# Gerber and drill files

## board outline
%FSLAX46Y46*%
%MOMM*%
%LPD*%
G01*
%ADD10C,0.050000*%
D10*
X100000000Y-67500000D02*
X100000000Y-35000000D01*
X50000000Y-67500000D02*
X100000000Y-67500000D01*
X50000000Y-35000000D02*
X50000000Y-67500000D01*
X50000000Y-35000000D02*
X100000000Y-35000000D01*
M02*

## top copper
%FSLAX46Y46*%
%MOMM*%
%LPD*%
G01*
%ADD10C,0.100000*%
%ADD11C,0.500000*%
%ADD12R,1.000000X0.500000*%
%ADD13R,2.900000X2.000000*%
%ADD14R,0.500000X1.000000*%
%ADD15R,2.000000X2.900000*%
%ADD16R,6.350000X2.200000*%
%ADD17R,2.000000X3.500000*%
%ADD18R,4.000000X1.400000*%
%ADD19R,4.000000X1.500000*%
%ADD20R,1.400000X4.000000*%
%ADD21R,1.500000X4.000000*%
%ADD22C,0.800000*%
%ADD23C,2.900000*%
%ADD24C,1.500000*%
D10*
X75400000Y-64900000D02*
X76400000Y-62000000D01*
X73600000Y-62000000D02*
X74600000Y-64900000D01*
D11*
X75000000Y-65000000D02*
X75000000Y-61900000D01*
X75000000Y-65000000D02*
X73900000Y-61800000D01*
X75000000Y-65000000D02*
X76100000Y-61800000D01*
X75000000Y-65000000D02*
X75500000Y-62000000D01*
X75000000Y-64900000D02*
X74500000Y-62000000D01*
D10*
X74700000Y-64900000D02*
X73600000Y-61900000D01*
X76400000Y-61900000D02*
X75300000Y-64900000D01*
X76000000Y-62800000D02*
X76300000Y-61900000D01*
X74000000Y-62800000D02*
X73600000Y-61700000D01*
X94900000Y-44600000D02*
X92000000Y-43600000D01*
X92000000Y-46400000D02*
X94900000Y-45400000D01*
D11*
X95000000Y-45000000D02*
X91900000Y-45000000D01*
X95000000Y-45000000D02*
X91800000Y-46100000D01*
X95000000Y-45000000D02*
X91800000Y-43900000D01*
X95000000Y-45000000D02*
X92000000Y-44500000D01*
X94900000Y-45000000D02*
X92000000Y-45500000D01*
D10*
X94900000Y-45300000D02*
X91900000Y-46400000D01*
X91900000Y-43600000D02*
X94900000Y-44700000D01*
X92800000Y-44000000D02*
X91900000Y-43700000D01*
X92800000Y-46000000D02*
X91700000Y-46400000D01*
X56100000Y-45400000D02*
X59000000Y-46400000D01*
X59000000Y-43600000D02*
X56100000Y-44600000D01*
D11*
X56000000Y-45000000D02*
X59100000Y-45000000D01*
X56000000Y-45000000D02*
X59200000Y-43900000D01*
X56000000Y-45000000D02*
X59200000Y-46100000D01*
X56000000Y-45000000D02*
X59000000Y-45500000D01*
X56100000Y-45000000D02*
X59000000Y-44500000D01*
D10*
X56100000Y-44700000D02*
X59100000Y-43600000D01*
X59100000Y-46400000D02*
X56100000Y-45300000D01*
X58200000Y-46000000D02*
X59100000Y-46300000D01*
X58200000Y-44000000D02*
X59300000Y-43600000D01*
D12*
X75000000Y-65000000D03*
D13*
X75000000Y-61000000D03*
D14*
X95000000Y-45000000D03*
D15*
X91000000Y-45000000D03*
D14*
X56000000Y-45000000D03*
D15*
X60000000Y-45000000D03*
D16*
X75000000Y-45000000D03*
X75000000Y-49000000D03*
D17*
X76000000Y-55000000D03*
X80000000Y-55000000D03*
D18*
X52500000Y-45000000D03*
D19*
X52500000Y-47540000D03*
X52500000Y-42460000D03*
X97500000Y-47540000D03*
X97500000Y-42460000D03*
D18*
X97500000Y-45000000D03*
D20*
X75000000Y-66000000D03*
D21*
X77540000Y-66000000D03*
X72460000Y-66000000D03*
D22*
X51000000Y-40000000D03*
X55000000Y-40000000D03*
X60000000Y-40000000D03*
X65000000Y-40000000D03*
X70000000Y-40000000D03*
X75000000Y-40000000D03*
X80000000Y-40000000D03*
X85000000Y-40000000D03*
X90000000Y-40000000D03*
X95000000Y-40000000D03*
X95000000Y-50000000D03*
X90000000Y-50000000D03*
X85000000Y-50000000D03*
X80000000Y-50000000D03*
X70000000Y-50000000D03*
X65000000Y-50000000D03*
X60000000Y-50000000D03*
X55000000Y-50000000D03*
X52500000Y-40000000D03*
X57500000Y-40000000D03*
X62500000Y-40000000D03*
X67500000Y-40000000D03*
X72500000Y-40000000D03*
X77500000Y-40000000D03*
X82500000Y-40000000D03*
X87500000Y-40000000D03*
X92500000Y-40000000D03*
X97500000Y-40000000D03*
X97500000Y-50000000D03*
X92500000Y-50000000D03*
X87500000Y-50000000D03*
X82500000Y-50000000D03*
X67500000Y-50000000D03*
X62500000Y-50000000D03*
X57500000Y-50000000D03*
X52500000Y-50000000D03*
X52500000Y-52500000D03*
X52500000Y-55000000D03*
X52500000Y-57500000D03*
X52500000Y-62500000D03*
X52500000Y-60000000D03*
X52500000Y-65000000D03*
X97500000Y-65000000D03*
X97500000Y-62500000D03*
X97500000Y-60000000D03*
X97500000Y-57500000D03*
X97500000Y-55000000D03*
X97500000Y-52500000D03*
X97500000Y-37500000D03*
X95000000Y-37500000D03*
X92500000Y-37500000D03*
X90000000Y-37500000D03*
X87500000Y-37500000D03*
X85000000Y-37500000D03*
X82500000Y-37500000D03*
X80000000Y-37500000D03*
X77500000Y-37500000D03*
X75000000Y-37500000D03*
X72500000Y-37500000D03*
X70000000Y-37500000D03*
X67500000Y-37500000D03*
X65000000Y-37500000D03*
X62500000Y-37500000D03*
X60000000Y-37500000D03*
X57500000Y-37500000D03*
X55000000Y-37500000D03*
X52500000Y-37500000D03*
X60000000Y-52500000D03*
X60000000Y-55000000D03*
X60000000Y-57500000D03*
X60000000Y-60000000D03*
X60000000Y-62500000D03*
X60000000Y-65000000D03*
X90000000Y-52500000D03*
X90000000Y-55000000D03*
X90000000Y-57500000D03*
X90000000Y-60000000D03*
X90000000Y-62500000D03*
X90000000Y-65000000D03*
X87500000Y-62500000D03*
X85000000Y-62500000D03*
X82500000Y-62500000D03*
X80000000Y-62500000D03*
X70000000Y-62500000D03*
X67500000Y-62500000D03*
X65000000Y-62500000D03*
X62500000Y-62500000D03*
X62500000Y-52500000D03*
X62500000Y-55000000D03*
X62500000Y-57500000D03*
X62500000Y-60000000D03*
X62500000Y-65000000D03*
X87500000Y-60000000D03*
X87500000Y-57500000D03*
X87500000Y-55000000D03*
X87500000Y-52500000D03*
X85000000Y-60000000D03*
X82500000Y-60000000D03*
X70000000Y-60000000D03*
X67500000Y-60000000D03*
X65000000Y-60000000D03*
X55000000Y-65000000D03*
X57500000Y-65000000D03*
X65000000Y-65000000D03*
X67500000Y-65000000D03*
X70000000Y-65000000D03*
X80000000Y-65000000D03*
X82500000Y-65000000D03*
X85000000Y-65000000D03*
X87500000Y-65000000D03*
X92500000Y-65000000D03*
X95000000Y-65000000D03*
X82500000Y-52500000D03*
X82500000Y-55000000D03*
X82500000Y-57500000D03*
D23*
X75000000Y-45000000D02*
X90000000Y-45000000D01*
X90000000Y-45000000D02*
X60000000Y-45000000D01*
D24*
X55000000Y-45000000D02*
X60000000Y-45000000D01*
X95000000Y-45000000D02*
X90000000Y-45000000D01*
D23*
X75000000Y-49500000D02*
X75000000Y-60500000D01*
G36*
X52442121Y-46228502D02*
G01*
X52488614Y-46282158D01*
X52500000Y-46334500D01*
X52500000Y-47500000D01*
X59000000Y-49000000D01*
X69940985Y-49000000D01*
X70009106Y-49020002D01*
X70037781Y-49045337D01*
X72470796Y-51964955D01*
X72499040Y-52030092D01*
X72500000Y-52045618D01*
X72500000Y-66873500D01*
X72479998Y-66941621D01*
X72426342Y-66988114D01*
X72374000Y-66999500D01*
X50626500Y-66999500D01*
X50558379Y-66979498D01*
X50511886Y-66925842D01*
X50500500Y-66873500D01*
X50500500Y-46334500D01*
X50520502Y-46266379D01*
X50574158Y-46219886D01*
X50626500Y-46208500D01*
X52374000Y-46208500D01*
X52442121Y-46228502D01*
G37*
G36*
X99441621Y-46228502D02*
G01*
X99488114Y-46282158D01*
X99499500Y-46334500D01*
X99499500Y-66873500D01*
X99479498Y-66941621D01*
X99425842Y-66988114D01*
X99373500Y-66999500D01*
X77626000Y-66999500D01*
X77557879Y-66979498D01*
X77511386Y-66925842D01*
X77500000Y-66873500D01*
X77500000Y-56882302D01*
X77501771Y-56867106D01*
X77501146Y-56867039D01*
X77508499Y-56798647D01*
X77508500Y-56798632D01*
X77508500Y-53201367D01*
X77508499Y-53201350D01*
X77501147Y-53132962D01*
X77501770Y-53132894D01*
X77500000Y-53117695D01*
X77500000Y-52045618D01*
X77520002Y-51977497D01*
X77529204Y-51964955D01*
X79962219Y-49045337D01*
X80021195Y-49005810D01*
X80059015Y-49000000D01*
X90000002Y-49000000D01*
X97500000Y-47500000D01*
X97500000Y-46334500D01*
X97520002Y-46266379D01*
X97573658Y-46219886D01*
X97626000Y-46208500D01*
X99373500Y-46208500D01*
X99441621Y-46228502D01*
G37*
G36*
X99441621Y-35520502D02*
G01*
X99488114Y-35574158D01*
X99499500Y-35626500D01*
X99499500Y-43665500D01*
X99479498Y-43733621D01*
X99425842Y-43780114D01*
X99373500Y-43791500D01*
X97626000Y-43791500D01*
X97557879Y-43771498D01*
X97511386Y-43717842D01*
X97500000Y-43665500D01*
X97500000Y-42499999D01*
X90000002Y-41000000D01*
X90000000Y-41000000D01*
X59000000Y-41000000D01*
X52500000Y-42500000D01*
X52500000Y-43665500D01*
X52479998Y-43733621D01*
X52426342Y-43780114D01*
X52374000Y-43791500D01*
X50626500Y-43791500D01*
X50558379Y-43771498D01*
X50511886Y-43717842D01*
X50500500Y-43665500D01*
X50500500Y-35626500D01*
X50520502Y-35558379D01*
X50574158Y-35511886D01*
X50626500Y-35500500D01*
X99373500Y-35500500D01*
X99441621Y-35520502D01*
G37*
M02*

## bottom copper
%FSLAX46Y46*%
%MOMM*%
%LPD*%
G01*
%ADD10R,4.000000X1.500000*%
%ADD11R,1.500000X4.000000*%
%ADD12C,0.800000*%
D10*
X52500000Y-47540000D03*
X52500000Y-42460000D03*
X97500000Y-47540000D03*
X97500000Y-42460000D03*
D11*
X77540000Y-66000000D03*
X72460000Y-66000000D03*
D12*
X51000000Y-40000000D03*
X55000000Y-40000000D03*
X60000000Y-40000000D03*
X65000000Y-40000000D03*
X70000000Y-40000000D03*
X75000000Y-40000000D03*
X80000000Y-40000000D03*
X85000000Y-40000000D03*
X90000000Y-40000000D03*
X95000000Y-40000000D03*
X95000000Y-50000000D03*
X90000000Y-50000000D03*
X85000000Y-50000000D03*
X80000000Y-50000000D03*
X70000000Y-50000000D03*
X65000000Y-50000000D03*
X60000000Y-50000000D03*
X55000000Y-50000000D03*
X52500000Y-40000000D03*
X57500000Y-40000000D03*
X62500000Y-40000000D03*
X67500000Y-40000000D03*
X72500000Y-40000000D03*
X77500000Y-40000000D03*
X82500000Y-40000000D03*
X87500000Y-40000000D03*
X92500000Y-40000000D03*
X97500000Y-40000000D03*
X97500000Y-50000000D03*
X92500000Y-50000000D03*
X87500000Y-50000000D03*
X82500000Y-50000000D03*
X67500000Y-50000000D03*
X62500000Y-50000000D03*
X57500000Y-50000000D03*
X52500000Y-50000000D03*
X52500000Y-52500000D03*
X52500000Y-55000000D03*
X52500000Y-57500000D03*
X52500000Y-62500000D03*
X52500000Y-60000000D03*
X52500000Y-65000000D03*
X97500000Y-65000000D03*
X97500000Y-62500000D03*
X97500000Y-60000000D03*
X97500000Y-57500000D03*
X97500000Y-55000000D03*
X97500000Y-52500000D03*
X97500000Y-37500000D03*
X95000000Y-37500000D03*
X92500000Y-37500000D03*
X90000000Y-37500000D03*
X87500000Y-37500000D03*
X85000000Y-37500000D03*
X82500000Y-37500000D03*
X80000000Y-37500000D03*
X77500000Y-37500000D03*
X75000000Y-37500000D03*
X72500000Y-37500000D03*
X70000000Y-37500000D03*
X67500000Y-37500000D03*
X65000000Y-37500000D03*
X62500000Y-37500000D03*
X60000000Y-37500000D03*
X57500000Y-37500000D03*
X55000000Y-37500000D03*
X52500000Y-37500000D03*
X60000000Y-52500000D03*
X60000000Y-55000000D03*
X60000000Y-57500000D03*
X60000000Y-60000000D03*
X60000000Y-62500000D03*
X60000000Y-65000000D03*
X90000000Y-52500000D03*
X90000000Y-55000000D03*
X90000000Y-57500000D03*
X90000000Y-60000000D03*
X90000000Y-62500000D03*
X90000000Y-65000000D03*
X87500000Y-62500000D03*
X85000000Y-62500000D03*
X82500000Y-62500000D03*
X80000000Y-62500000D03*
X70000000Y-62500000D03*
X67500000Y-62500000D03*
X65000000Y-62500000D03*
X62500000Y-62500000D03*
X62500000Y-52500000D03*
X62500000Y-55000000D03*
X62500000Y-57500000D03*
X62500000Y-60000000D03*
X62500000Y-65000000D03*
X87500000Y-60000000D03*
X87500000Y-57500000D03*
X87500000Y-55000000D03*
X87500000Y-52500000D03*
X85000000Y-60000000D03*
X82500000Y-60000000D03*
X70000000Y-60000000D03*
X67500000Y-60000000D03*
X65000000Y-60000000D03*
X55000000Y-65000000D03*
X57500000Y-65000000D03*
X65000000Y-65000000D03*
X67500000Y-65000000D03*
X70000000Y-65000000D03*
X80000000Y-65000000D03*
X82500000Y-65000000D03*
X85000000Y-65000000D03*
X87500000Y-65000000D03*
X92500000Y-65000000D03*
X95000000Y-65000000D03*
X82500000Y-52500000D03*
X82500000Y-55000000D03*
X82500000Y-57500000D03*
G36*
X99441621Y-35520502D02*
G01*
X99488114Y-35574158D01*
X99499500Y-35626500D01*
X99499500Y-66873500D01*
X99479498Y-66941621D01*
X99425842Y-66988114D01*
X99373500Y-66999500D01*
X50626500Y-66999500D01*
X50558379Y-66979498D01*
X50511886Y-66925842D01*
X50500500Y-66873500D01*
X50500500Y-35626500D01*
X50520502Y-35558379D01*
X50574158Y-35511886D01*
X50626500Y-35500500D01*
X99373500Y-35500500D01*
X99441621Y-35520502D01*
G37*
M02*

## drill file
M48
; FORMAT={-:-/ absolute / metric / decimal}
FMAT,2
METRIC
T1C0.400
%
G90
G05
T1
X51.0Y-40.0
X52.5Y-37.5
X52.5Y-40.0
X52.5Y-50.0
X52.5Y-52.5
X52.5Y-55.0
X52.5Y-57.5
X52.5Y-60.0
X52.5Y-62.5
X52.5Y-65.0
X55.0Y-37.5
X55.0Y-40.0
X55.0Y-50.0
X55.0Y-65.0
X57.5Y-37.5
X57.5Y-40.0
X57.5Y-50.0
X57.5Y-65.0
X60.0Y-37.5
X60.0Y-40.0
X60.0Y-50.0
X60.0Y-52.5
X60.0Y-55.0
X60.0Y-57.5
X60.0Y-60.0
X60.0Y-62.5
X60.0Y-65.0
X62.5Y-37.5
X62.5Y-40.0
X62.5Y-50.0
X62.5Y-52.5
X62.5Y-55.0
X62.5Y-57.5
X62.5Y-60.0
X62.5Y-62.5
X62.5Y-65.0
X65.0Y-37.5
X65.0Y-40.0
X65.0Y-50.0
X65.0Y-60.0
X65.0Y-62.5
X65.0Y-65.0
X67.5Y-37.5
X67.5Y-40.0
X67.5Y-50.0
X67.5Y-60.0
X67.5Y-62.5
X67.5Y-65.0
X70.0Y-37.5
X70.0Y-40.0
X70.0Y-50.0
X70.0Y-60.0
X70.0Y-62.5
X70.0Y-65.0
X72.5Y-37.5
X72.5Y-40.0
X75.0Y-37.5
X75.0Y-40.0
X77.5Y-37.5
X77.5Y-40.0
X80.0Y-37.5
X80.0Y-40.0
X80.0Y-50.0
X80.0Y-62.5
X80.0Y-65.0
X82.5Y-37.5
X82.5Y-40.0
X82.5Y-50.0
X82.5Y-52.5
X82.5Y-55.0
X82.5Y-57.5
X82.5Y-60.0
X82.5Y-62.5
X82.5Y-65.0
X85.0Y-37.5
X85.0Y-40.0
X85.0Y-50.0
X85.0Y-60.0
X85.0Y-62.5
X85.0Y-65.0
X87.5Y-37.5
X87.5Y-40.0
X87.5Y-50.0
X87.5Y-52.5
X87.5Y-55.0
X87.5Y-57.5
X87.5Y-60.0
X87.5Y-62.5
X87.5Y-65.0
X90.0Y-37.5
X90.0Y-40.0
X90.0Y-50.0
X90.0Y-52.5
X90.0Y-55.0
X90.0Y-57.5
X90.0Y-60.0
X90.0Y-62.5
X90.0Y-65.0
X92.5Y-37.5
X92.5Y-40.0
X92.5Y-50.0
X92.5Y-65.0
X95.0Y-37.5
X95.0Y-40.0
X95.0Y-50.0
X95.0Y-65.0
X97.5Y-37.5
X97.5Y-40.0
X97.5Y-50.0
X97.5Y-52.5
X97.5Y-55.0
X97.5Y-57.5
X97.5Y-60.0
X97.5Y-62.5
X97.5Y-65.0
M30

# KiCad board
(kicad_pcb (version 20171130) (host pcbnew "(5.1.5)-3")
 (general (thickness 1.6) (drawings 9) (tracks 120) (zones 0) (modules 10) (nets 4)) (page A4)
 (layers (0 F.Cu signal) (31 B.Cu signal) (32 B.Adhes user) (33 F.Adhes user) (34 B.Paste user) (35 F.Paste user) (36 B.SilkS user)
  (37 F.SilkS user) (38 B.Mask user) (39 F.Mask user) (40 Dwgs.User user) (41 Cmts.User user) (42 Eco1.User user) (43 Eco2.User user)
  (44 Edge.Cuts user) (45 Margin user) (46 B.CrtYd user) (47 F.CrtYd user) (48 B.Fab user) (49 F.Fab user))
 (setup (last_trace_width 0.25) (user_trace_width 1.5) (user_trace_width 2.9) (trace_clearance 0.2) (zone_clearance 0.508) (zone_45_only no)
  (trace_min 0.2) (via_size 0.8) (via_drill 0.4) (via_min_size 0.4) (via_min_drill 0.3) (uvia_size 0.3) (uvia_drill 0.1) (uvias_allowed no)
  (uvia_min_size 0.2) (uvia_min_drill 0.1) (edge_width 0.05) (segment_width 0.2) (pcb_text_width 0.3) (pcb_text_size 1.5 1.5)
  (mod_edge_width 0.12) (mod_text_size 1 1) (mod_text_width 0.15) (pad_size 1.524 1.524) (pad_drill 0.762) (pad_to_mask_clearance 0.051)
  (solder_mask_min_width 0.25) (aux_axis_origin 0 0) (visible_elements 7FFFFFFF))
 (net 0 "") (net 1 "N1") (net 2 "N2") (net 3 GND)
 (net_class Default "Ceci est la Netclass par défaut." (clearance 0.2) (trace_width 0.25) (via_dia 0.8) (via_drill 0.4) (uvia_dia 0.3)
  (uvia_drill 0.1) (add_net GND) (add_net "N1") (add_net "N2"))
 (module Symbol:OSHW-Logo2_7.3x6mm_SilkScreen (layer B.Cu) (at 86.4 56.4 180)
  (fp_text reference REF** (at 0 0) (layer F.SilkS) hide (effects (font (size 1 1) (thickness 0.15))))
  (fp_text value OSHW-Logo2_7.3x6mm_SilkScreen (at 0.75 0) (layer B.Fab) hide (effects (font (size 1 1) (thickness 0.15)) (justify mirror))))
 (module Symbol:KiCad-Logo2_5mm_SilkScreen (layer B.Cu) (at 66.9 56.4 180)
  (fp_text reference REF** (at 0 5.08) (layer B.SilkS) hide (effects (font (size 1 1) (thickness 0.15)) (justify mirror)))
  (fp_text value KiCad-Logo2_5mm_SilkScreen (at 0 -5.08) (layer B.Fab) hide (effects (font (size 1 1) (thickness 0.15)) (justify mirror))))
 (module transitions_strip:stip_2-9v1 (layer F.Cu) (at 75 63 270)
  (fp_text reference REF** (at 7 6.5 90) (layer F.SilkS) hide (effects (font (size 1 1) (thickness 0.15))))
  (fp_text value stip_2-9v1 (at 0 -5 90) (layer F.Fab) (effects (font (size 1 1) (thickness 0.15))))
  (fp_line (start 1.9 -0.4) (end -1 -1.4) (layer F.Cu) (width 0.1))
  (fp_line (start -1 1.4) (end 1.9 0.4) (layer F.Cu) (width 0.1)) (fp_line (start 2 0) (end -1.1 0) (layer F.Cu) (width 0.5))
  (fp_line (start 2 0) (end -1.2 1.1) (layer F.Cu) (width 0.5))
  (fp_line (start 2 0) (end -1.2 -1.1) (layer F.Cu) (width 0.5)) (fp_line (start 2 0) (end -1 -0.5) (layer F.Cu) (width 0.5))
  (fp_line (start 1.9 0) (end -1 0.5) (layer F.Cu) (width 0.5))
  (fp_line (start 1.9 0.3) (end -1.1 1.4) (layer F.Cu) (width 0.1))
  (fp_line (start -1.1 -1.4) (end 1.9 -0.3) (layer F.Cu) (width 0.1))
  (fp_line (start -0.2 -1) (end -1.1 -1.3) (layer F.Cu) (width 0.1))
  (fp_line (start -0.2 1) (end -1.3 1.4) (layer F.Cu) (width 0.1))
  (pad 2 smd rect (at 2 0 270) (size 0.5 1) (layers F.Cu F.Paste F.Mask))
  (pad 1 smd rect (at -2 0 270) (size 2 2.9) (layers F.Cu F.Paste F.Mask)))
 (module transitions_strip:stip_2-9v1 (layer F.Cu) (at 93 45)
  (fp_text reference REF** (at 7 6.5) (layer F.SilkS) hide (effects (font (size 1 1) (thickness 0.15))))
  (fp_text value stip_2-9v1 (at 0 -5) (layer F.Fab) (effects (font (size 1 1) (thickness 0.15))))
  (fp_line (start 1.9 -0.4) (end -1 -1.4) (layer F.Cu) (width 0.1))
  (fp_line (start -1 1.4) (end 1.9 0.4) (layer F.Cu) (width 0.1)) (fp_line (start 2 0) (end -1.1 0) (layer F.Cu) (width 0.5))
  (fp_line (start 2 0) (end -1.2 1.1) (layer F.Cu) (width 0.5))
  (fp_line (start 2 0) (end -1.2 -1.1) (layer F.Cu) (width 0.5)) (fp_line (start 2 0) (end -1 -0.5) (layer F.Cu) (width 0.5))
  (fp_line (start 1.9 0) (end -1 0.5) (layer F.Cu) (width 0.5))
  (fp_line (start 1.9 0.3) (end -1.1 1.4) (layer F.Cu) (width 0.1))
  (fp_line (start -1.1 -1.4) (end 1.9 -0.3) (layer F.Cu) (width 0.1))
  (fp_line (start -0.2 -1) (end -1.1 -1.3) (layer F.Cu) (width 0.1))
  (fp_line (start -0.2 1) (end -1.3 1.4) (layer F.Cu) (width 0.1))
  (pad 2 smd rect (at 2 0) (size 0.5 1) (layers F.Cu F.Paste F.Mask))
  (pad 1 smd rect (at -2 0) (size 2 2.9) (layers F.Cu F.Paste F.Mask)))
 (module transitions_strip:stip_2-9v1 (layer F.Cu) (at 58 45 180)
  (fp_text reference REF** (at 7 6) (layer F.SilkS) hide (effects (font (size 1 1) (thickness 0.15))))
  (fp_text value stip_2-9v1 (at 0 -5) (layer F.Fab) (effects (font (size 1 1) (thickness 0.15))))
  (fp_line (start 1.9 -0.4) (end -1 -1.4) (layer F.Cu) (width 0.1))
  (fp_line (start -1 1.4) (end 1.9 0.4) (layer F.Cu) (width 0.1)) (fp_line (start 2 0) (end -1.1 0) (layer F.Cu) (width 0.5))
  (fp_line (start 2 0) (end -1.2 1.1) (layer F.Cu) (width 0.5))
  (fp_line (start 2 0) (end -1.2 -1.1) (layer F.Cu) (width 0.5)) (fp_line (start 2 0) (end -1 -0.5) (layer F.Cu) (width 0.5))
  (fp_line (start 1.9 0) (end -1 0.5) (layer F.Cu) (width 0.5))
  (fp_line (start 1.9 0.3) (end -1.1 1.4) (layer F.Cu) (width 0.1))
  (fp_line (start -1.1 -1.4) (end 1.9 -0.3) (layer F.Cu) (width 0.1))
  (fp_line (start -0.2 -1) (end -1.1 -1.3) (layer F.Cu) (width 0.1))
  (fp_line (start -0.2 1) (end -1.3 1.4) (layer F.Cu) (width 0.1))
  (pad 2 smd rect (at 2 0 180) (size 0.5 1) (layers F.Cu F.Paste F.Mask))
  (pad 1 smd rect (at -2 0 180) (size 2 2.9) (layers F.Cu F.Paste F.Mask)))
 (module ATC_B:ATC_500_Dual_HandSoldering (layer F.Cu) (at 75 47 270)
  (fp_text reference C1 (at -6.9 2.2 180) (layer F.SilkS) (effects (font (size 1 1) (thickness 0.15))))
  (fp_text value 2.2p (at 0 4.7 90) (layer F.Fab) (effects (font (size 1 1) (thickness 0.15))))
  (pad 1 smd rect (at -2 0 270) (size 2.2 6.35) (layers F.Cu F.Paste F.Mask) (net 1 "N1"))
  (pad 2 smd rect (at 2 0 270) (size 2.2 6.35) (layers F.Cu F.Paste F.Mask) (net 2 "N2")))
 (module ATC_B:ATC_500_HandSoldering (layer F.Cu) (at 78 55)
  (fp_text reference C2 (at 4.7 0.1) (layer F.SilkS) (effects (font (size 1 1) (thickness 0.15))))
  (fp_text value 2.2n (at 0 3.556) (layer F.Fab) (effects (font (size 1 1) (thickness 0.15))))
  (pad 1 smd rect (at -2 0) (size 2 3.5) (layers F.Cu F.Paste F.Mask) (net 2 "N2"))
  (pad 2 smd rect (at 2 0) (size 2 3.5) (layers F.Cu F.Paste F.Mask) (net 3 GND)))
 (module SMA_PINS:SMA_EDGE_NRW (layer F.Cu) (at 52.5 45 180)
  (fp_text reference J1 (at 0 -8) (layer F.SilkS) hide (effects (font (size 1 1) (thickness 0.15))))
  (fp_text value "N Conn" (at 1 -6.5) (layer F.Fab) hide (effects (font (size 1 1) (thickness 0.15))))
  (pad 1 smd rect (at 0 0 180) (size 4 1.4) (layers F.Cu F.Paste F.Mask) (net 1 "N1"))
  (pad 2 smd rect (at 0 -2.54 180) (size 4 1.5) (layers F.Cu F.Paste F.Mask) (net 3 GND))
  (pad 2 smd rect (at 0 2.54 180) (size 4 1.5) (layers F.Cu F.Paste F.Mask) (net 3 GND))
  (pad 2 smd rect (at 0 -2.54 180) (size 4 1.5) (layers B.Cu B.Paste B.Mask) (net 3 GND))
  (pad 2 smd rect (at 0 2.54 180) (size 4 1.5) (layers B.Cu B.Paste B.Mask) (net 3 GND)))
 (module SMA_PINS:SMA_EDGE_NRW (layer F.Cu) (at 97.5 45)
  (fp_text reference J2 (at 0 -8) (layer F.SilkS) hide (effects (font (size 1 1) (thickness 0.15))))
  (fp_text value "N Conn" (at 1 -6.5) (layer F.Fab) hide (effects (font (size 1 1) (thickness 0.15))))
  (pad 2 smd rect (at 0 2.54) (size 4 1.5) (layers B.Cu B.Paste B.Mask) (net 3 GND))
  (pad 2 smd rect (at 0 -2.54) (size 4 1.5) (layers B.Cu B.Paste B.Mask) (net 3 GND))
  (pad 2 smd rect (at 0 2.54) (size 4 1.5) (layers F.Cu F.Paste F.Mask) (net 3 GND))
  (pad 2 smd rect (at 0 -2.54) (size 4 1.5) (layers F.Cu F.Paste F.Mask) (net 3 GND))
  (pad 1 smd rect (at 0 0) (size 4 1.4) (layers F.Cu F.Paste F.Mask) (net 1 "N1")))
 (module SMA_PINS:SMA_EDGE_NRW (layer F.Cu) (at 75 66 270)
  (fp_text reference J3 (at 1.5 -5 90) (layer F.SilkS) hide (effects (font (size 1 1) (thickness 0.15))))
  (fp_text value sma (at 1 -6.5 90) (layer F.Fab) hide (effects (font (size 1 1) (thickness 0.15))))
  (pad 1 smd rect (at 0 0 270) (size 4 1.4) (layers F.Cu F.Paste F.Mask) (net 2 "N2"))
  (pad 2 smd rect (at 0 -2.54 270) (size 4 1.5) (layers F.Cu F.Paste F.Mask) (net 3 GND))
  (pad 2 smd rect (at 0 2.54 270) (size 4 1.5) (layers F.Cu F.Paste F.Mask) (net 3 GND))
  (pad 2 smd rect (at 0 -2.54 270) (size 4 1.5) (layers B.Cu B.Paste B.Mask) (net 3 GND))
  (pad 2 smd rect (at 0 2.54 270) (size 4 1.5) (layers B.Cu B.Paste B.Mask) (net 3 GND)))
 (gr_line (start 100 67.5) (end 100 35) (layer Edge.Cuts) (width 0.05))
 (gr_line (start 50 67.5) (end 100 67.5) (layer Edge.Cuts) (width 0.05))
 (gr_line (start 50 35) (end 50 67.5) (layer Edge.Cuts) (width 0.05))
 (gr_line (start 50 35) (end 100 35) (layer Edge.Cuts) (width 0.05))
 (segment (start 75 45) (end 90 45) (width 2.9) (layer F.Cu) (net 1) (status 10))
 (segment (start 90 45) (end 60 45) (width 2.9) (layer F.Cu) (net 1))
 (segment (start 55 45) (end 60 45) (width 1.5) (layer F.Cu) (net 1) (status 10))
 (segment (start 95 45) (end 90 45) (width 1.5) (layer F.Cu) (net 1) (status 10))
 (segment (start 75 49.5) (end 75 60.5) (width 2.9) (layer F.Cu) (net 2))
 (via (at 51 40) (size 0.8) (drill 0.4) (layers F.Cu B.Cu) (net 3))
 (via (at 55 40) (size 0.8) (drill 0.4) (layers F.Cu B.Cu) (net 3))
 (via (at 60 40) (size 0.8) (drill 0.4) (layers F.Cu B.Cu) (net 3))
 (via (at 65 40) (size 0.8) (drill 0.4) (layers F.Cu B.Cu) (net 3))
 (via (at 70 40) (size 0.8) (drill 0.4) (layers F.Cu B.Cu) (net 3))
 (via (at 75 40) (size 0.8) (drill 0.4) (layers F.Cu B.Cu) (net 3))
 (via (at 80 40) (size 0.8) (drill 0.4) (layers F.Cu B.Cu) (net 3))
 (via (at 85 40) (size 0.8) (drill 0.4) (layers F.Cu B.Cu) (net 3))
 (via (at 90 40) (size 0.8) (drill 0.4) (layers F.Cu B.Cu) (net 3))
 (via (at 95 40) (size 0.8) (drill 0.4) (layers F.Cu B.Cu) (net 3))
 (via (at 95 50) (size 0.8) (drill 0.4) (layers F.Cu B.Cu) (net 3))
 (via (at 90 50) (size 0.8) (drill 0.4) (layers F.Cu B.Cu) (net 3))
 (via (at 85 50) (size 0.8) (drill 0.4) (layers F.Cu B.Cu) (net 3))
 (via (at 80 50) (size 0.8) (drill 0.4) (layers F.Cu B.Cu) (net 3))
 (via (at 70 50) (size 0.8) (drill 0.4) (layers F.Cu B.Cu) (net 3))
 (via (at 65 50) (size 0.8) (drill 0.4) (layers F.Cu B.Cu) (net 3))
 (via (at 60 50) (size 0.8) (drill 0.4) (layers F.Cu B.Cu) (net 3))
 (via (at 55 50) (size 0.8) (drill 0.4) (layers F.Cu B.Cu) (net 3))
 (via (at 52.5 40) (size 0.8) (drill 0.4) (layers F.Cu B.Cu) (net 3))
 (via (at 57.5 40) (size 0.8) (drill 0.4) (layers F.Cu B.Cu) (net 3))
 (via (at 62.5 40) (size 0.8) (drill 0.4) (layers F.Cu B.Cu) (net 3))
 (via (at 67.5 40) (size 0.8) (drill 0.4) (layers F.Cu B.Cu) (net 3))
 (via (at 72.5 40) (size 0.8) (drill 0.4) (layers F.Cu B.Cu) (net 3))
 (via (at 77.5 40) (size 0.8) (drill 0.4) (layers F.Cu B.Cu) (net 3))
 (via (at 82.5 40) (size 0.8) (drill 0.4) (layers F.Cu B.Cu) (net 3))
 (via (at 87.5 40) (size 0.8) (drill 0.4) (layers F.Cu B.Cu) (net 3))
 (via (at 92.5 40) (size 0.8) (drill 0.4) (layers F.Cu B.Cu) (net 3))
 (via (at 97.5 40) (size 0.8) (drill 0.4) (layers F.Cu B.Cu) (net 3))
 (via (at 97.5 50) (size 0.8) (drill 0.4) (layers F.Cu B.Cu) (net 3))
 (via (at 92.5 50) (size 0.8) (drill 0.4) (layers F.Cu B.Cu) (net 3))
 (via (at 87.5 50) (size 0.8) (drill 0.4) (layers F.Cu B.Cu) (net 3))
 (via (at 82.5 50) (size 0.8) (drill 0.4) (layers F.Cu B.Cu) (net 3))
 (via (at 67.5 50) (size 0.8) (drill 0.4) (layers F.Cu B.Cu) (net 3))
 (via (at 62.5 50) (size 0.8) (drill 0.4) (layers F.Cu B.Cu) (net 3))
 (via (at 57.5 50) (size 0.8) (drill 0.4) (layers F.Cu B.Cu) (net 3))
 (via (at 52.5 50) (size 0.8) (drill 0.4) (layers F.Cu B.Cu) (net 3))
 (via (at 52.5 52.5) (size 0.8) (drill 0.4) (layers F.Cu B.Cu) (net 3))
 (via (at 52.5 55) (size 0.8) (drill 0.4) (layers F.Cu B.Cu) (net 3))
 (via (at 52.5 57.5) (size 0.8) (drill 0.4) (layers F.Cu B.Cu) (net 3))
 (via (at 52.5 62.5) (size 0.8) (drill 0.4) (layers F.Cu B.Cu) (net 3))
 (via (at 52.5 60) (size 0.8) (drill 0.4) (layers F.Cu B.Cu) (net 3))
 (via (at 52.5 65) (size 0.8) (drill 0.4) (layers F.Cu B.Cu) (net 3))
 (via (at 97.5 65) (size 0.8) (drill 0.4) (layers F.Cu B.Cu) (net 3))
 (via (at 97.5 62.5) (size 0.8) (drill 0.4) (layers F.Cu B.Cu) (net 3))
 (via (at 97.5 60) (size 0.8) (drill 0.4) (layers F.Cu B.Cu) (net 3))
 (via (at 97.5 57.5) (size 0.8) (drill 0.4) (layers F.Cu B.Cu) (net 3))
 (via (at 97.5 55) (size 0.8) (drill 0.4) (layers F.Cu B.Cu) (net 3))
 (via (at 97.5 52.5) (size 0.8) (drill 0.4) (layers F.Cu B.Cu) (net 3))
 (via (at 97.5 37.5) (size 0.8) (drill 0.4) (layers F.Cu B.Cu) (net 3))
 (via (at 95 37.5) (size 0.8) (drill 0.4) (layers F.Cu B.Cu) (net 3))
 (via (at 92.5 37.5) (size 0.8) (drill 0.4) (layers F.Cu B.Cu) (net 3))
 (via (at 90 37.5) (size 0.8) (drill 0.4) (layers F.Cu B.Cu) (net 3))
 (via (at 87.5 37.5) (size 0.8) (drill 0.4) (layers F.Cu B.Cu) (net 3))
 (via (at 85 37.5) (size 0.8) (drill 0.4) (layers F.Cu B.Cu) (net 3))
 (via (at 82.5 37.5) (size 0.8) (drill 0.4) (layers F.Cu B.Cu) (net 3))
 (via (at 80 37.5) (size 0.8) (drill 0.4) (layers F.Cu B.Cu) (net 3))
 (via (at 77.5 37.5) (size 0.8) (drill 0.4) (layers F.Cu B.Cu) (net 3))
 (via (at 75 37.5) (size 0.8) (drill 0.4) (layers F.Cu B.Cu) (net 3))
 (via (at 72.5 37.5) (size 0.8) (drill 0.4) (layers F.Cu B.Cu) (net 3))
 (via (at 70 37.5) (size 0.8) (drill 0.4) (layers F.Cu B.Cu) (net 3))
 (via (at 67.5 37.5) (size 0.8) (drill 0.4) (layers F.Cu B.Cu) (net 3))
 (via (at 65 37.5) (size 0.8) (drill 0.4) (layers F.Cu B.Cu) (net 3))
 (via (at 62.5 37.5) (size 0.8) (drill 0.4) (layers F.Cu B.Cu) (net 3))
 (via (at 60 37.5) (size 0.8) (drill 0.4) (layers F.Cu B.Cu) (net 3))
 (via (at 57.5 37.5) (size 0.8) (drill 0.4) (layers F.Cu B.Cu) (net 3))
 (via (at 55 37.5) (size 0.8) (drill 0.4) (layers F.Cu B.Cu) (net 3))
 (via (at 52.5 37.5) (size 0.8) (drill 0.4) (layers F.Cu B.Cu) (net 3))
 (via (at 60 52.5) (size 0.8) (drill 0.4) (layers F.Cu B.Cu) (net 3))
 (via (at 60 55) (size 0.8) (drill 0.4) (layers F.Cu B.Cu) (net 3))
 (via (at 60 57.5) (size 0.8) (drill 0.4) (layers F.Cu B.Cu) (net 3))
 (via (at 60 60) (size 0.8) (drill 0.4) (layers F.Cu B.Cu) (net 3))
 (via (at 60 62.5) (size 0.8) (drill 0.4) (layers F.Cu B.Cu) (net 3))
 (via (at 60 65) (size 0.8) (drill 0.4) (layers F.Cu B.Cu) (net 3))
 (via (at 90 52.5) (size 0.8) (drill 0.4) (layers F.Cu B.Cu) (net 3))
 (via (at 90 55) (size 0.8) (drill 0.4) (layers F.Cu B.Cu) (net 3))
 (via (at 90 57.5) (size 0.8) (drill 0.4) (layers F.Cu B.Cu) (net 3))
 (via (at 90 60) (size 0.8) (drill 0.4) (layers F.Cu B.Cu) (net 3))
 (via (at 90 62.5) (size 0.8) (drill 0.4) (layers F.Cu B.Cu) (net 3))
 (via (at 90 65) (size 0.8) (drill 0.4) (layers F.Cu B.Cu) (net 3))
 (via (at 87.5 62.5) (size 0.8) (drill 0.4) (layers F.Cu B.Cu) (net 3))
 (via (at 85 62.5) (size 0.8) (drill 0.4) (layers F.Cu B.Cu) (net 3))
 (via (at 82.5 62.5) (size 0.8) (drill 0.4) (layers F.Cu B.Cu) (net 3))
 (via (at 80 62.5) (size 0.8) (drill 0.4) (layers F.Cu B.Cu) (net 3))
 (via (at 70 62.5) (size 0.8) (drill 0.4) (layers F.Cu B.Cu) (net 3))
 (via (at 67.5 62.5) (size 0.8) (drill 0.4) (layers F.Cu B.Cu) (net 3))
 (via (at 65 62.5) (size 0.8) (drill 0.4) (layers F.Cu B.Cu) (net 3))
 (via (at 62.5 62.5) (size 0.8) (drill 0.4) (layers F.Cu B.Cu) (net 3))
 (via (at 62.5 52.5) (size 0.8) (drill 0.4) (layers F.Cu B.Cu) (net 3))
 (via (at 62.5 55) (size 0.8) (drill 0.4) (layers F.Cu B.Cu) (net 3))
 (via (at 62.5 57.5) (size 0.8) (drill 0.4) (layers F.Cu B.Cu) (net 3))
 (via (at 62.5 60) (size 0.8) (drill 0.4) (layers F.Cu B.Cu) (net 3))
 (via (at 62.5 65) (size 0.8) (drill 0.4) (layers F.Cu B.Cu) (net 3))
 (via (at 87.5 60) (size 0.8) (drill 0.4) (layers F.Cu B.Cu) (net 3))
 (via (at 87.5 57.5) (size 0.8) (drill 0.4) (layers F.Cu B.Cu) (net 3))
 (via (at 87.5 55) (size 0.8) (drill 0.4) (layers F.Cu B.Cu) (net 3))
 (via (at 87.5 52.5) (size 0.8) (drill 0.4) (layers F.Cu B.Cu) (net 3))
 (via (at 85 60) (size 0.8) (drill 0.4) (layers F.Cu B.Cu) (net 3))
 (via (at 82.5 60) (size 0.8) (drill 0.4) (layers F.Cu B.Cu) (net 3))
 (via (at 70 60) (size 0.8) (drill 0.4) (layers F.Cu B.Cu) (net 3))
 (via (at 67.5 60) (size 0.8) (drill 0.4) (layers F.Cu B.Cu) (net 3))
 (via (at 65 60) (size 0.8) (drill 0.4) (layers F.Cu B.Cu) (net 3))
 (via (at 55 65) (size 0.8) (drill 0.4) (layers F.Cu B.Cu) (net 3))
 (via (at 57.5 65) (size 0.8) (drill 0.4) (layers F.Cu B.Cu) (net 3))
 (via (at 65 65) (size 0.8) (drill 0.4) (layers F.Cu B.Cu) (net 3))
 (via (at 67.5 65) (size 0.8) (drill 0.4) (layers F.Cu B.Cu) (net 3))
 (via (at 70 65) (size 0.8) (drill 0.4) (layers F.Cu B.Cu) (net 3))
 (via (at 80 65) (size 0.8) (drill 0.4) (layers F.Cu B.Cu) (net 3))
 (via (at 82.5 65) (size 0.8) (drill 0.4) (layers F.Cu B.Cu) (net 3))
 (via (at 85 65) (size 0.8) (drill 0.4) (layers F.Cu B.Cu) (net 3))
 (via (at 87.5 65) (size 0.8) (drill 0.4) (layers F.Cu B.Cu) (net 3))
 (via (at 92.5 65) (size 0.8) (drill 0.4) (layers F.Cu B.Cu) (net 3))
 (via (at 95 65) (size 0.8) (drill 0.4) (layers F.Cu B.Cu) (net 3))
 (via (at 82.5 52.5) (size 0.8) (drill 0.4) (layers F.Cu B.Cu) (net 3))
 (via (at 82.5 55) (size 0.8) (drill 0.4) (layers F.Cu B.Cu) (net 3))
 (via (at 82.5 57.5) (size 0.8) (drill 0.4) (layers F.Cu B.Cu) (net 3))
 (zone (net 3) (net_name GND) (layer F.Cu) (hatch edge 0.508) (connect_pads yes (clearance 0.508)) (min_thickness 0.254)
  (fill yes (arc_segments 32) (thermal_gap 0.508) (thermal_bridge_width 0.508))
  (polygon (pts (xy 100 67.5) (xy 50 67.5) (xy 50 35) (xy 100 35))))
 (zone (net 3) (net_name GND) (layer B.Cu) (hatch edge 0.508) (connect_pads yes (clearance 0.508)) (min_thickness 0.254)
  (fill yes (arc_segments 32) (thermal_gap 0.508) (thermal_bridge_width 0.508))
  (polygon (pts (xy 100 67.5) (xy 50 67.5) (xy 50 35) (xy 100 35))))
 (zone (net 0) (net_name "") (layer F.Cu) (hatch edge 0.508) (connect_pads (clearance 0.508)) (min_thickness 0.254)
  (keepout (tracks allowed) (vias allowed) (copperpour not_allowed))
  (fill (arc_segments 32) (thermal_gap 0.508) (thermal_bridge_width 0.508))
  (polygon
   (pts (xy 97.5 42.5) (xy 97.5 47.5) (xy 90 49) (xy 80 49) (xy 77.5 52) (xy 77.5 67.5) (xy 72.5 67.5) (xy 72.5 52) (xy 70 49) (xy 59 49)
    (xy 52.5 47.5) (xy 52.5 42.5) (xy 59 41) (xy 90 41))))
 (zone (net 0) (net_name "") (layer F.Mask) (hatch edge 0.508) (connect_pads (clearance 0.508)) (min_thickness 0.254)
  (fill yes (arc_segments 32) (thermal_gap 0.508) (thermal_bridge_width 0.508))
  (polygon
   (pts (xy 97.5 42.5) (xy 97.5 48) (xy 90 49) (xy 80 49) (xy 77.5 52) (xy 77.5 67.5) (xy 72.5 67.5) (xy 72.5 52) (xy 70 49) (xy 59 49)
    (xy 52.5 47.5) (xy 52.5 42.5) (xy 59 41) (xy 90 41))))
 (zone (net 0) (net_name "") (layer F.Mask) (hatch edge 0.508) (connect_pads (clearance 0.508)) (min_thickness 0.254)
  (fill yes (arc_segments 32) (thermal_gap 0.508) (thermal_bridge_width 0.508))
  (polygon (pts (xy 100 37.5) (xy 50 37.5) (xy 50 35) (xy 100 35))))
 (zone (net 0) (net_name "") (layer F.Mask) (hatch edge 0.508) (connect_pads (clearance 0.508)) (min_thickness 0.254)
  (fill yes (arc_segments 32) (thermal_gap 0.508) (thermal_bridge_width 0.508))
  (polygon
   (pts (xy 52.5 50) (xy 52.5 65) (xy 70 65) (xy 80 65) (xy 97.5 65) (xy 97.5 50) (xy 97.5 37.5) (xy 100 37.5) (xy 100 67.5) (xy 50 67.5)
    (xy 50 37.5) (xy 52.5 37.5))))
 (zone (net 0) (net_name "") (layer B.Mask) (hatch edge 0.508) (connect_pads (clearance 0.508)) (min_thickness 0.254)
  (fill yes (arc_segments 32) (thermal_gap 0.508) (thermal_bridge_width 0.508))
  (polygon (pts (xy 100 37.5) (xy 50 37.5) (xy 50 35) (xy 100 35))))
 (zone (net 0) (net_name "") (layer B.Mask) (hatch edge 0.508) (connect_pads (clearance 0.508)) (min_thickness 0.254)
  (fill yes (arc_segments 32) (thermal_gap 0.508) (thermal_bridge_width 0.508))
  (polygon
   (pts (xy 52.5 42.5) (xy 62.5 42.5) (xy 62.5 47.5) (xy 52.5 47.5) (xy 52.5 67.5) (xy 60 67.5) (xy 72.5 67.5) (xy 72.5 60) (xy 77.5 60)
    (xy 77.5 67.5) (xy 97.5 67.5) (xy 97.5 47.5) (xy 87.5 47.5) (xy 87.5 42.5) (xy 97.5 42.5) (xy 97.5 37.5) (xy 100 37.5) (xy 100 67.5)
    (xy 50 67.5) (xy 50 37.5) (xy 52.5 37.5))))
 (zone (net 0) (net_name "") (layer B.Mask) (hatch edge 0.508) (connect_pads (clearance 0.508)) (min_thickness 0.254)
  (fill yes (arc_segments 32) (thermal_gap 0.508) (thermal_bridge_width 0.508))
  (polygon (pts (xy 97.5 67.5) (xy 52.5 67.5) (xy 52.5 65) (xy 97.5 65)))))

